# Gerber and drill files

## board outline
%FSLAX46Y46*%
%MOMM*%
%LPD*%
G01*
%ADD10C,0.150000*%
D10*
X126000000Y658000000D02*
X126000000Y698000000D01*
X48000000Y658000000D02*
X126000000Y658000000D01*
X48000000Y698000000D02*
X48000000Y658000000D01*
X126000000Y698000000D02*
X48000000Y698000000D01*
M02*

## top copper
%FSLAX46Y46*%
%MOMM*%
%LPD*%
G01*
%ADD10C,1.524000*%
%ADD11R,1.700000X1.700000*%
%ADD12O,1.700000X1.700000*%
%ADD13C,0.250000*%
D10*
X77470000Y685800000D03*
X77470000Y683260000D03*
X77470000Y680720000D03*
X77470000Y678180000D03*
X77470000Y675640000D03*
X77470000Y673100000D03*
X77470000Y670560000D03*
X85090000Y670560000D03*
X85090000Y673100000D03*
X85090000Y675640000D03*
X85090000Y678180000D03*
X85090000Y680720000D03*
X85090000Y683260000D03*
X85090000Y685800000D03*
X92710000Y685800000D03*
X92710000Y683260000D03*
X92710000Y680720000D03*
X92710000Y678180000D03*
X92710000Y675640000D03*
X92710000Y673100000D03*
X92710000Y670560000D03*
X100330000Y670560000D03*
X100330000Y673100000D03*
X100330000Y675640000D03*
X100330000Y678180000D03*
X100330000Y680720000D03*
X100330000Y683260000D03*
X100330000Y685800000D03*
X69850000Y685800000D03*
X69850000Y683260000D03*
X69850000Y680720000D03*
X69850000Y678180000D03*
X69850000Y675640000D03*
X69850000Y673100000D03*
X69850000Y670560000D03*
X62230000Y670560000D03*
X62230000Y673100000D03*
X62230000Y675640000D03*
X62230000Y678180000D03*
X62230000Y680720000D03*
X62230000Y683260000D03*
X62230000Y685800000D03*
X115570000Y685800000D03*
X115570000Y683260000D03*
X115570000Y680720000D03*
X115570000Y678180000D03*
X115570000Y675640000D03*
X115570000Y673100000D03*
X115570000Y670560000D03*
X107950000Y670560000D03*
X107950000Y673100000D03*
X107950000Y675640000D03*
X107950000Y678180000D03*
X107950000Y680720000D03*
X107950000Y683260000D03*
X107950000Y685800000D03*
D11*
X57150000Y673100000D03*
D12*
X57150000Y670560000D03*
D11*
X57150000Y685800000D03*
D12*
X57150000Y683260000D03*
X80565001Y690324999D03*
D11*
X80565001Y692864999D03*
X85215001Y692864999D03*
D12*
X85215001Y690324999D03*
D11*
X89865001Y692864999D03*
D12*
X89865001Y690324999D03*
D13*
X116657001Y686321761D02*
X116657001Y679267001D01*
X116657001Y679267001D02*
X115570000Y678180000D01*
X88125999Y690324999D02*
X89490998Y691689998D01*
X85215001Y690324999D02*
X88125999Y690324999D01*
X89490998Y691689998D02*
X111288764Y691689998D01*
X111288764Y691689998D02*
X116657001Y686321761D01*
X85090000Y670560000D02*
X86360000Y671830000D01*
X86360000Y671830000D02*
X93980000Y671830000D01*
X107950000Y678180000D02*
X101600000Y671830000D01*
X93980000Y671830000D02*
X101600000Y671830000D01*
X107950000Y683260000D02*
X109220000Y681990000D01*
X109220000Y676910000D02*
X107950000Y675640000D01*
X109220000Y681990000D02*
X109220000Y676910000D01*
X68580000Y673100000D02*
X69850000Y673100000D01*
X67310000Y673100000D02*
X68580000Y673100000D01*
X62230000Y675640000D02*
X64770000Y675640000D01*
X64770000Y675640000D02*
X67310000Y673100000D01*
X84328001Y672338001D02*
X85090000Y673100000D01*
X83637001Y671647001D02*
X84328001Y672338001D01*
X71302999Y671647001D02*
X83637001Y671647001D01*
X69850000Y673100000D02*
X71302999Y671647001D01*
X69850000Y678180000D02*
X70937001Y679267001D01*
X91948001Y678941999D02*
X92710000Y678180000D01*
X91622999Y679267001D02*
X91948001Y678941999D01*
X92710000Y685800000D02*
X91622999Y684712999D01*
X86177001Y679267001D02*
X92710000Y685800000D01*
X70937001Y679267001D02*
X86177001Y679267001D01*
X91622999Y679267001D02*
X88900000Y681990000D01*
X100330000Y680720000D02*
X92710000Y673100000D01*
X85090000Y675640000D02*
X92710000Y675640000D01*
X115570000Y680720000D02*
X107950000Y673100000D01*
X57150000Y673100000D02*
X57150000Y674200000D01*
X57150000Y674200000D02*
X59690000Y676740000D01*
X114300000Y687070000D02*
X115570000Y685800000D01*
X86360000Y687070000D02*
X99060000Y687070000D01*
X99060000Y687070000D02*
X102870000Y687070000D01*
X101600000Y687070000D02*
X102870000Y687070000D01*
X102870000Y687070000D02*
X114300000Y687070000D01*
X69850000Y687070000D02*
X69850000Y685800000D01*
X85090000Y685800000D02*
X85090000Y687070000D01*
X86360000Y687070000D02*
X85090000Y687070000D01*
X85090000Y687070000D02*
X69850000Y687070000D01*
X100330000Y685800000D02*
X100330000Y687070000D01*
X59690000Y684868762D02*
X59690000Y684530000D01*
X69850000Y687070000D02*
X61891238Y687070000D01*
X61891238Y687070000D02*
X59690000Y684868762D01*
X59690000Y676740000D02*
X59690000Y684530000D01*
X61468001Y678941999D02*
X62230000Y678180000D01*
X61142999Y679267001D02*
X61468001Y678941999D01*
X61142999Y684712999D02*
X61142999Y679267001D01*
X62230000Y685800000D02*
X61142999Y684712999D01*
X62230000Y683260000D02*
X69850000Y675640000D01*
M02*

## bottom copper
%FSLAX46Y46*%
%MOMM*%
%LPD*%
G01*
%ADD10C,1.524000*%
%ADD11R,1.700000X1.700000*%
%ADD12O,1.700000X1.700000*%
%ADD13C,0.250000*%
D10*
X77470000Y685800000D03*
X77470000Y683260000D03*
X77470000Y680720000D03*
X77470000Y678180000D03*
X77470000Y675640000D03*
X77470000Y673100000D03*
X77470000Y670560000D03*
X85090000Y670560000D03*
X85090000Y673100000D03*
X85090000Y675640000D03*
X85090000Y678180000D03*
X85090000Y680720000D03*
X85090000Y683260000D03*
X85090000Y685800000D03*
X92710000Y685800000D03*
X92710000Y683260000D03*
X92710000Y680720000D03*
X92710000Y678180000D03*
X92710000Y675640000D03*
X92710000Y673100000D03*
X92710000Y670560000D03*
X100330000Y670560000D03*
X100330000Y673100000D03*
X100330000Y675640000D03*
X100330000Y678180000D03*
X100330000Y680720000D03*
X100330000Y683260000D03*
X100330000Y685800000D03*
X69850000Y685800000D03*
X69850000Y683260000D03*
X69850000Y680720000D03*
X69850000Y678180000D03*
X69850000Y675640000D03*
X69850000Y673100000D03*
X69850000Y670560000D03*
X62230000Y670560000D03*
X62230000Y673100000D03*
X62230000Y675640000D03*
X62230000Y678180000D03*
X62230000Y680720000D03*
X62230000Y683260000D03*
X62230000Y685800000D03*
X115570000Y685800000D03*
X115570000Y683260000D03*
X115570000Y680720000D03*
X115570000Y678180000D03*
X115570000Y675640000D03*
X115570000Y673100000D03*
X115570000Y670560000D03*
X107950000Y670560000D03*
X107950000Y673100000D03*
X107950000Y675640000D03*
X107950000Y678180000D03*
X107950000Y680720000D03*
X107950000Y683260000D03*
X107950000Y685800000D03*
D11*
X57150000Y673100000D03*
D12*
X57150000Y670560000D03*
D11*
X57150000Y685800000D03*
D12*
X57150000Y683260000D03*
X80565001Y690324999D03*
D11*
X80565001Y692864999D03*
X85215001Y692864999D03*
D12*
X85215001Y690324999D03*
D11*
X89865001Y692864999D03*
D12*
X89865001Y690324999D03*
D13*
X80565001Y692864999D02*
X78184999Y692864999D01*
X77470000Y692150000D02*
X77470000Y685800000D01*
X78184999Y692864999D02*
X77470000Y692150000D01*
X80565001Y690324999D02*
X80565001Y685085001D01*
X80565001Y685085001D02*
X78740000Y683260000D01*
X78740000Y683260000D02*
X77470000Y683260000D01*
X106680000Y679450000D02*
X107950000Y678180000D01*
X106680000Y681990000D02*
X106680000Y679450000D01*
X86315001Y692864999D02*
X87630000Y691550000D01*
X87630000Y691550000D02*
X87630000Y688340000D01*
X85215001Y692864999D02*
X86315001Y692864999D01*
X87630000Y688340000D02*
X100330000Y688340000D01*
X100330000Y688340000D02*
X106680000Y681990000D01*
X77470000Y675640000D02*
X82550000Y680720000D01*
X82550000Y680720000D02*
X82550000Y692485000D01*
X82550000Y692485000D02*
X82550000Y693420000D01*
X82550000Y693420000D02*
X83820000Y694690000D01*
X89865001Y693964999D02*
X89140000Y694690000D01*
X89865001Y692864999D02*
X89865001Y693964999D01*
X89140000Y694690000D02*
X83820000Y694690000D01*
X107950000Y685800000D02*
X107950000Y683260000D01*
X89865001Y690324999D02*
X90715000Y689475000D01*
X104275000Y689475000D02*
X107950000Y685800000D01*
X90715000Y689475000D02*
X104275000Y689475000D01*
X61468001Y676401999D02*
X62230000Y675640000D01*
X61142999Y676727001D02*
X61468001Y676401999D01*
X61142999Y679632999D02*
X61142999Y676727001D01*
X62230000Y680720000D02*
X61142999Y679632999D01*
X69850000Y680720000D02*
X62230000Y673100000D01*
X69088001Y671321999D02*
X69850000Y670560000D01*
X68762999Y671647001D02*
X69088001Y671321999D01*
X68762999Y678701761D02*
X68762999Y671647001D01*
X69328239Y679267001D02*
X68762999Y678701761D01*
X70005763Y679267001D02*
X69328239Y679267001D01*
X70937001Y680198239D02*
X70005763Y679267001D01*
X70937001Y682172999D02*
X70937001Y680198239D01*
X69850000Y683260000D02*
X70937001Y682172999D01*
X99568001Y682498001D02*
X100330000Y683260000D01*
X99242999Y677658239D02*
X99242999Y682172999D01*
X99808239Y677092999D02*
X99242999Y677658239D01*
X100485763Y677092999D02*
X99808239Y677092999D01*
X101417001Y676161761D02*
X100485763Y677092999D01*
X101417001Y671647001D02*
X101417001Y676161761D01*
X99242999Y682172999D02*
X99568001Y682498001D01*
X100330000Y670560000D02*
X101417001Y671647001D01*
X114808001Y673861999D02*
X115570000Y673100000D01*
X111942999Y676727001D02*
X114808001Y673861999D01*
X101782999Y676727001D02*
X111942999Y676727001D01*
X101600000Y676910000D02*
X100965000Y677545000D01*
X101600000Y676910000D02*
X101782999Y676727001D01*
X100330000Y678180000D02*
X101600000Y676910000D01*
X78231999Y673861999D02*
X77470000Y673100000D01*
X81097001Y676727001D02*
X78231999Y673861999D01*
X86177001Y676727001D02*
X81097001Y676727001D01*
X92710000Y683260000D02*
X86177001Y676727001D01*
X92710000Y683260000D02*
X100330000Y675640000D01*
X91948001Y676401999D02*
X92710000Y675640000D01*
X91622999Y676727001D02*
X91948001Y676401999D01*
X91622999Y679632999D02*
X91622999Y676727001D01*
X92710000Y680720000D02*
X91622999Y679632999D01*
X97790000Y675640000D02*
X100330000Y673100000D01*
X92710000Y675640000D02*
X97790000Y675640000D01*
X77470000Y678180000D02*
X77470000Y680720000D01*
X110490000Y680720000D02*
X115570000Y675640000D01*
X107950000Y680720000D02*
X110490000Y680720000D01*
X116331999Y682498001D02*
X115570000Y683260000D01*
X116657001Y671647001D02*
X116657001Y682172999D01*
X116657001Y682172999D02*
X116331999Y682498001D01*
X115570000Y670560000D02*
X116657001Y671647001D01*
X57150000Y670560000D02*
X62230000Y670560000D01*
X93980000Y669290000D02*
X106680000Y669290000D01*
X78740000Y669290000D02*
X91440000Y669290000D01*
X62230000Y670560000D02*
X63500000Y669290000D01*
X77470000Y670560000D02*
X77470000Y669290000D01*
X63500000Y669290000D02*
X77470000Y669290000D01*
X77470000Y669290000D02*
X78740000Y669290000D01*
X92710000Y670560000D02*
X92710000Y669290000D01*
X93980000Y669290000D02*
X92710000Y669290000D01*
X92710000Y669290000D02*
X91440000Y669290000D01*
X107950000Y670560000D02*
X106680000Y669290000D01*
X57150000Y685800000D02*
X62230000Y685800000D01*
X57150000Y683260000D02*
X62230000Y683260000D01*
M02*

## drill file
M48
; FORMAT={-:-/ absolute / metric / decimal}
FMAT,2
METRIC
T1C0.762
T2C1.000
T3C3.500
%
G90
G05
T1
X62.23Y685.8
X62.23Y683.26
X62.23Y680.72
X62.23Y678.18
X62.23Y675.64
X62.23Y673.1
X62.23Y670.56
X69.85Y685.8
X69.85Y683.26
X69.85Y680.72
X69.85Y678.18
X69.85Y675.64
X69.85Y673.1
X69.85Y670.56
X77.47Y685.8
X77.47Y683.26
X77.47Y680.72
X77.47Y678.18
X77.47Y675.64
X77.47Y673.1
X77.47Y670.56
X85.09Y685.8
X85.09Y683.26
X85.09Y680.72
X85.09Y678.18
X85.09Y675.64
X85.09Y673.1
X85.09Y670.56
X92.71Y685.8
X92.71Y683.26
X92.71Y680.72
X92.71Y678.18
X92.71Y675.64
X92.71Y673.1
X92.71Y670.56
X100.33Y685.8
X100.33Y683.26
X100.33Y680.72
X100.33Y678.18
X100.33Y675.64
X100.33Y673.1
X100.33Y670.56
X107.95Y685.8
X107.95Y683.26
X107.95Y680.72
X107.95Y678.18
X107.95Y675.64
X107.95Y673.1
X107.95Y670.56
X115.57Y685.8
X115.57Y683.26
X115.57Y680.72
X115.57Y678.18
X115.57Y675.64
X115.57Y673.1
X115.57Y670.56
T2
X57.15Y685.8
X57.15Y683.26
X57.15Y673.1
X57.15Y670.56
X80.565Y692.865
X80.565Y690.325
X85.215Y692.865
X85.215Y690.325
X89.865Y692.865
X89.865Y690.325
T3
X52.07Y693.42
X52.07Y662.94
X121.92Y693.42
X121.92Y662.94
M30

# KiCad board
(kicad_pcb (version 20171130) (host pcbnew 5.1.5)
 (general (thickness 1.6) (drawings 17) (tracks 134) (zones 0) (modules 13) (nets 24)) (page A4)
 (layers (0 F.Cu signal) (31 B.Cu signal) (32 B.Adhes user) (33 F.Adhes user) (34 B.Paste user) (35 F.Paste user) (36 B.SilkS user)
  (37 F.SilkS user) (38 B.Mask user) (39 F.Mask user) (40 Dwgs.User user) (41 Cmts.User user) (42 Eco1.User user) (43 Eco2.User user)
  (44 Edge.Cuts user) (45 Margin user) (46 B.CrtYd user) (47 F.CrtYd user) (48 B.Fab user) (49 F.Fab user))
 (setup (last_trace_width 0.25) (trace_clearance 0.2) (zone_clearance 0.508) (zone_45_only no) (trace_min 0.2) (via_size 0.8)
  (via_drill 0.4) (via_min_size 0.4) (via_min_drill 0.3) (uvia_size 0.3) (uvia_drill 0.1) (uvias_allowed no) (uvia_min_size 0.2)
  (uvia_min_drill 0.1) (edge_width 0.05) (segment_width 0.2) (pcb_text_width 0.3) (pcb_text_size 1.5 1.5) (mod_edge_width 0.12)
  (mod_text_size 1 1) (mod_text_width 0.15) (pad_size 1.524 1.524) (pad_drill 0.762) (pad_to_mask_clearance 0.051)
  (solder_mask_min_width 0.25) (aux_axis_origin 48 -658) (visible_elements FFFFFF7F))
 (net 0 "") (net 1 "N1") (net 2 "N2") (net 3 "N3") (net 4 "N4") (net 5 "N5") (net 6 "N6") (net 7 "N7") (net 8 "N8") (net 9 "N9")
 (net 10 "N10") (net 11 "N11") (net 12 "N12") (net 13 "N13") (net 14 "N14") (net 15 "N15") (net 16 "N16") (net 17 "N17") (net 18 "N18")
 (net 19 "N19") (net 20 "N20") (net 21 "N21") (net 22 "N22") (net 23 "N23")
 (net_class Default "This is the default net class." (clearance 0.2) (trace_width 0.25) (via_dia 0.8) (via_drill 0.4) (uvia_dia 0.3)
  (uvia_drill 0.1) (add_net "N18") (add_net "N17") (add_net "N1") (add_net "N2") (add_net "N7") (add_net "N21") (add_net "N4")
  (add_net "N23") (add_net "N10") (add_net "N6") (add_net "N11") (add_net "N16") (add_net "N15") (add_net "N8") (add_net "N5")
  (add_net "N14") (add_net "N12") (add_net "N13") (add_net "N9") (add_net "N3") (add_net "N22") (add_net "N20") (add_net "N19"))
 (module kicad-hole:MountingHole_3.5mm (layer F.Cu) (at 121.92 -662.94)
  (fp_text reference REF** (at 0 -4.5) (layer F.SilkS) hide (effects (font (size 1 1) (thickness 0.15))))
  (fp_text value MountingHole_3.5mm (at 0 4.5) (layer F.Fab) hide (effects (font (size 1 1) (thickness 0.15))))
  (pad 1 np_thru_hole circle (at 0 0) (size 3.5 3.5) (drill 3.5) (layers *.Cu *.Mask)))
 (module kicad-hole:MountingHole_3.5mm (layer F.Cu) (at 52.07 -693.42)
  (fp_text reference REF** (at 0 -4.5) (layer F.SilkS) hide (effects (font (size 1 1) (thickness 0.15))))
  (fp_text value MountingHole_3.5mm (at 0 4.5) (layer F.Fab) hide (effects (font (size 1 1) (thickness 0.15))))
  (pad 1 np_thru_hole circle (at 0 0) (size 3.5 3.5) (drill 3.5) (layers *.Cu *.Mask)))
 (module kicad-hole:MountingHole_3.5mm (layer F.Cu) (at 52.07 -662.94)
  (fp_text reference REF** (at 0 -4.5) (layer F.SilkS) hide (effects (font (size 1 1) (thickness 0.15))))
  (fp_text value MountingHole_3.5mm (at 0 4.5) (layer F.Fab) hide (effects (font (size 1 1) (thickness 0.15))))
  (pad 1 np_thru_hole circle (at 0 0) (size 3.5 3.5) (drill 3.5) (layers *.Cu *.Mask)))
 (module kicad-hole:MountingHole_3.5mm (layer F.Cu) (at 121.92 -693.42)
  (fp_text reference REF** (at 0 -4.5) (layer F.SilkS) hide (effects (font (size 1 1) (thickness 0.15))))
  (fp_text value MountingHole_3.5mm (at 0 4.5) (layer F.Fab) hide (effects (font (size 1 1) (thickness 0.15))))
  (pad 1 np_thru_hole circle (at 0 0) (size 3.5 3.5) (drill 3.5) (layers *.Cu *.Mask)))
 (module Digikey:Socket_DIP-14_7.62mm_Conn (layer F.Cu) (at 77.47 -685.8)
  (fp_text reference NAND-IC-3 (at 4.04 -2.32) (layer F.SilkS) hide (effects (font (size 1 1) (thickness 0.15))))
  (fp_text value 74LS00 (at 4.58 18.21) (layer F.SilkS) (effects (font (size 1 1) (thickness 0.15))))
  (pad 1 thru_hole circle (at 0 0) (size 1.524 1.524) (drill 0.762) (layers *.Cu *.Mask) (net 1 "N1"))
  (pad 2 thru_hole circle (at 0 2.54) (size 1.524 1.524) (drill 0.762) (layers *.Cu *.Mask) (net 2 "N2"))
  (pad 3 thru_hole circle (at 0 5.08) (size 1.524 1.524) (drill 0.762) (layers *.Cu *.Mask) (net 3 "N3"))
  (pad 4 thru_hole circle (at 0 7.62) (size 1.524 1.524) (drill 0.762) (layers *.Cu *.Mask) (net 3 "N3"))
  (pad 5 thru_hole circle (at 0 10.16) (size 1.524 1.524) (drill 0.762) (layers *.Cu *.Mask) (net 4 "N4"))
  (pad 6 thru_hole circle (at 0 12.7) (size 1.524 1.524) (drill 0.762) (layers *.Cu *.Mask) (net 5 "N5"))
  (pad 7 thru_hole circle (at 0 15.24) (size 1.524 1.524) (drill 0.762) (layers *.Cu *.Mask) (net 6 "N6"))
  (pad 8 thru_hole circle (at 7.62 15.24) (size 1.524 1.524) (drill 0.762) (layers *.Cu *.Mask) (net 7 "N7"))
  (pad 9 thru_hole circle (at 7.62 12.7) (size 1.524 1.524) (drill 0.762) (layers *.Cu *.Mask) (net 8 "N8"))
  (pad 10 thru_hole circle (at 7.62 10.16) (size 1.524 1.524) (drill 0.762) (layers *.Cu *.Mask) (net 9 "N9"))
  (pad 11 thru_hole circle (at 7.62 7.62) (size 1.524 1.524) (drill 0.762) (layers *.Cu *.Mask))
  (pad 12 thru_hole circle (at 7.62 5.08) (size 1.524 1.524) (drill 0.762) (layers *.Cu *.Mask))
  (pad 13 thru_hole circle (at 7.62 2.54) (size 1.524 1.524) (drill 0.762) (layers *.Cu *.Mask))
  (pad 14 thru_hole circle (at 7.62 0) (size 1.524 1.524) (drill 0.762) (layers *.Cu *.Mask) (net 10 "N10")))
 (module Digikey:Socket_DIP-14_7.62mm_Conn (layer F.Cu) (at 92.71 -685.8)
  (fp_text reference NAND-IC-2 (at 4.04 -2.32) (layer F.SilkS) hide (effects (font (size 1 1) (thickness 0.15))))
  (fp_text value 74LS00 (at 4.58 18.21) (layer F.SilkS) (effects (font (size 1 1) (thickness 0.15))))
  (pad 1 thru_hole circle (at 0 0) (size 1.524 1.524) (drill 0.762) (layers *.Cu *.Mask) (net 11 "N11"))
  (pad 2 thru_hole circle (at 0 2.54) (size 1.524 1.524) (drill 0.762) (layers *.Cu *.Mask) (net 5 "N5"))
  (pad 3 thru_hole circle (at 0 5.08) (size 1.524 1.524) (drill 0.762) (layers *.Cu *.Mask) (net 9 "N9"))
  (pad 4 thru_hole circle (at 0 7.62) (size 1.524 1.524) (drill 0.762) (layers *.Cu *.Mask) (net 11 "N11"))
  (pad 5 thru_hole circle (at 0 10.16) (size 1.524 1.524) (drill 0.762) (layers *.Cu *.Mask) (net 9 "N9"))
  (pad 6 thru_hole circle (at 0 12.7) (size 1.524 1.524) (drill 0.762) (layers *.Cu *.Mask) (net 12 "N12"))
  (pad 7 thru_hole circle (at 0 15.24) (size 1.524 1.524) (drill 0.762) (layers *.Cu *.Mask) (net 6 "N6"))
  (pad 8 thru_hole circle (at 7.62 15.24) (size 1.524 1.524) (drill 0.762) (layers *.Cu *.Mask) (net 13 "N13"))
  (pad 9 thru_hole circle (at 7.62 12.7) (size 1.524 1.524) (drill 0.762) (layers *.Cu *.Mask) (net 9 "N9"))
  (pad 10 thru_hole circle (at 7.62 10.16) (size 1.524 1.524) (drill 0.762) (layers *.Cu *.Mask) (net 5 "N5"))
  (pad 11 thru_hole circle (at 7.62 7.62) (size 1.524 1.524) (drill 0.762) (layers *.Cu *.Mask) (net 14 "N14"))
  (pad 12 thru_hole circle (at 7.62 5.08) (size 1.524 1.524) (drill 0.762) (layers *.Cu *.Mask) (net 12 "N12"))
  (pad 13 thru_hole circle (at 7.62 2.54) (size 1.524 1.524) (drill 0.762) (layers *.Cu *.Mask) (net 13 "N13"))
  (pad 14 thru_hole circle (at 7.62 0) (size 1.524 1.524) (drill 0.762) (layers *.Cu *.Mask) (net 10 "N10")))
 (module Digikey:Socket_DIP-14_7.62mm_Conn (layer F.Cu) (at 62.23 -685.8)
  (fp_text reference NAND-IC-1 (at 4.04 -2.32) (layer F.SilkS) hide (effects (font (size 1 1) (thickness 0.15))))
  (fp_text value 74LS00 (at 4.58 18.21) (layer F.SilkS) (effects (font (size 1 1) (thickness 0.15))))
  (pad 14 thru_hole circle (at 7.62 0) (size 1.524 1.524) (drill 0.762) (layers *.Cu *.Mask) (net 10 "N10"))
  (pad 13 thru_hole circle (at 7.62 2.54) (size 1.524 1.524) (drill 0.762) (layers *.Cu *.Mask) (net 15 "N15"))
  (pad 12 thru_hole circle (at 7.62 5.08) (size 1.524 1.524) (drill 0.762) (layers *.Cu *.Mask) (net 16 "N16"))
  (pad 11 thru_hole circle (at 7.62 7.62) (size 1.524 1.524) (drill 0.762) (layers *.Cu *.Mask) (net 11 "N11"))
  (pad 10 thru_hole circle (at 7.62 10.16) (size 1.524 1.524) (drill 0.762) (layers *.Cu *.Mask) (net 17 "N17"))
  (pad 9 thru_hole circle (at 7.62 12.7) (size 1.524 1.524) (drill 0.762) (layers *.Cu *.Mask) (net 8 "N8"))
  (pad 8 thru_hole circle (at 7.62 15.24) (size 1.524 1.524) (drill 0.762) (layers *.Cu *.Mask) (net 15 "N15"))
  (pad 7 thru_hole circle (at 0 15.24) (size 1.524 1.524) (drill 0.762) (layers *.Cu *.Mask) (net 6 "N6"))
  (pad 6 thru_hole circle (at 0 12.7) (size 1.524 1.524) (drill 0.762) (layers *.Cu *.Mask) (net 16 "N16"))
  (pad 5 thru_hole circle (at 0 10.16) (size 1.524 1.524) (drill 0.762) (layers *.Cu *.Mask) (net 8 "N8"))
  (pad 4 thru_hole circle (at 0 7.62) (size 1.524 1.524) (drill 0.762) (layers *.Cu *.Mask) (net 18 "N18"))
  (pad 3 thru_hole circle (at 0 5.08) (size 1.524 1.524) (drill 0.762) (layers *.Cu *.Mask) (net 8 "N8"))
  (pad 2 thru_hole circle (at 0 2.54) (size 1.524 1.524) (drill 0.762) (layers *.Cu *.Mask) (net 17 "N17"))
  (pad 1 thru_hole circle (at 0 0) (size 1.524 1.524) (drill 0.762) (layers *.Cu *.Mask) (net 18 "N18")))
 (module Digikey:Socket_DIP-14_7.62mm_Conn (layer F.Cu) (at 107.95 -685.8)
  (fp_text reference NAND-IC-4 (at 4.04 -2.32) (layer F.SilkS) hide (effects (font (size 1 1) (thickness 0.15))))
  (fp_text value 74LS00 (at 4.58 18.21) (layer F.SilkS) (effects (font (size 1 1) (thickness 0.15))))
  (pad 14 thru_hole circle (at 7.62 0) (size 1.524 1.524) (drill 0.762) (layers *.Cu *.Mask) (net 10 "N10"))
  (pad 13 thru_hole circle (at 7.62 2.54) (size 1.524 1.524) (drill 0.762) (layers *.Cu *.Mask) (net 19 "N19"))
  (pad 12 thru_hole circle (at 7.62 5.08) (size 1.524 1.524) (drill 0.762) (layers *.Cu *.Mask) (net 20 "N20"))
  (pad 11 thru_hole circle (at 7.62 7.62) (size 1.524 1.524) (drill 0.762) (layers *.Cu *.Mask) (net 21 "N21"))
  (pad 10 thru_hole circle (at 7.62 10.16) (size 1.524 1.524) (drill 0.762) (layers *.Cu *.Mask) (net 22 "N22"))
  (pad 9 thru_hole circle (at 7.62 12.7) (size 1.524 1.524) (drill 0.762) (layers *.Cu *.Mask) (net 14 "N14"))
  (pad 8 thru_hole circle (at 7.62 15.24) (size 1.524 1.524) (drill 0.762) (layers *.Cu *.Mask) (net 19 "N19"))
  (pad 7 thru_hole circle (at 0 15.24) (size 1.524 1.524) (drill 0.762) (layers *.Cu *.Mask) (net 6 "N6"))
  (pad 6 thru_hole circle (at 0 12.7) (size 1.524 1.524) (drill 0.762) (layers *.Cu *.Mask) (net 20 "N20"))
  (pad 5 thru_hole circle (at 0 10.16) (size 1.524 1.524) (drill 0.762) (layers *.Cu *.Mask) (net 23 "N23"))
  (pad 4 thru_hole circle (at 0 7.62) (size 1.524 1.524) (drill 0.762) (layers *.Cu *.Mask) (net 7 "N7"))
  (pad 3 thru_hole circle (at 0 5.08) (size 1.524 1.524) (drill 0.762) (layers *.Cu *.Mask) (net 22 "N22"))
  (pad 2 thru_hole circle (at 0 2.54) (size 1.524 1.524) (drill 0.762) (layers *.Cu *.Mask) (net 23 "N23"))
  (pad 1 thru_hole circle (at 0 0) (size 1.524 1.524) (drill 0.762) (layers *.Cu *.Mask) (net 23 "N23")))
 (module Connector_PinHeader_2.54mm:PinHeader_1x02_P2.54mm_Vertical (layer F.Cu) (at 57.15 -673.1)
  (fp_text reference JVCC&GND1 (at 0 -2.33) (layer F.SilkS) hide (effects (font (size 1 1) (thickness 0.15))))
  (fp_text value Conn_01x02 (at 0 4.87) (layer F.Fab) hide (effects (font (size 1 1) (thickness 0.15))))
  (pad 1 thru_hole rect (at 0 0) (size 1.7 1.7) (drill 1) (layers *.Cu *.Mask) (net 10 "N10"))
  (pad 2 thru_hole oval (at 0 2.54) (size 1.7 1.7) (drill 1) (layers *.Cu *.Mask) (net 6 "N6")))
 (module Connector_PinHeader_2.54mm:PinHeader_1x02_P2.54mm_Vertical (layer F.Cu) (at 57.15 -685.8)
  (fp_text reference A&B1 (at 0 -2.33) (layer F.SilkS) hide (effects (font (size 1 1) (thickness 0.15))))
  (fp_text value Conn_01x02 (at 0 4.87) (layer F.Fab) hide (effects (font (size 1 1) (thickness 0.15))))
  (pad 1 thru_hole rect (at 0 0) (size 1.7 1.7) (drill 1) (layers *.Cu *.Mask) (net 18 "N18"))
  (pad 2 thru_hole oval (at 0 2.54) (size 1.7 1.7) (drill 1) (layers *.Cu *.Mask) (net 17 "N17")))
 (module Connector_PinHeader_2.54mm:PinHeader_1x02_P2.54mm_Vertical (layer F.Cu) (at 80.565001 -692.864999)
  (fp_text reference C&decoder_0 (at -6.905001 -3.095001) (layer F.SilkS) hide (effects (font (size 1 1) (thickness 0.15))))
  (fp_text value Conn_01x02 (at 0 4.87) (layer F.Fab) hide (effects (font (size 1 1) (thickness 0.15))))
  (pad 2 thru_hole oval (at 0 2.54) (size 1.7 1.7) (drill 1) (layers *.Cu *.Mask) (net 2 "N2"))
  (pad 1 thru_hole rect (at 0 0) (size 1.7 1.7) (drill 1) (layers *.Cu *.Mask) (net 1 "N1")))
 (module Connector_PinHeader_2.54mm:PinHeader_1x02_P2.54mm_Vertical (layer F.Cu) (at 85.215001 -692.864999)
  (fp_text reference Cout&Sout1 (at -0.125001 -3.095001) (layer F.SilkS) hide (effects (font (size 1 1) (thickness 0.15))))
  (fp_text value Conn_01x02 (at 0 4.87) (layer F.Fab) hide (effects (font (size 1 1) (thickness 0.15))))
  (pad 1 thru_hole rect (at 0 0) (size 1.7 1.7) (drill 1) (layers *.Cu *.Mask) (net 7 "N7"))
  (pad 2 thru_hole oval (at 0 2.54) (size 1.7 1.7) (drill 1) (layers *.Cu *.Mask) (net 21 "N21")))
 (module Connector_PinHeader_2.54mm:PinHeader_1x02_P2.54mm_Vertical (layer F.Cu) (at 89.865001 -692.864999)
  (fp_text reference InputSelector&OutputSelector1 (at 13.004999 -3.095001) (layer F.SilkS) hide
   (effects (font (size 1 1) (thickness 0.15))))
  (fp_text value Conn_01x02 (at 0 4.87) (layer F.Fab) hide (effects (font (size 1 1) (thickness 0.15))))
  (pad 1 thru_hole rect (at 0 0) (size 1.7 1.7) (drill 1) (layers *.Cu *.Mask) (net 4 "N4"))
  (pad 2 thru_hole oval (at 0 2.54) (size 1.7 1.7) (drill 1) (layers *.Cu *.Mask) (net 23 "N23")))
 (gr_line (start 126 -658) (end 126 -698) (layer Edge.Cuts) (width 0.15))
 (gr_line (start 48 -658) (end 126 -658) (layer Edge.Cuts) (width 0.15))
 (gr_line (start 48 -698) (end 48 -658) (layer Edge.Cuts) (width 0.15))
 (gr_line (start 126 -698) (end 48 -698) (layer Edge.Cuts) (width 0.15))
 (segment (start 80.565001 -692.864999) (end 78.184999 -692.864999) (width 0.25) (layer B.Cu) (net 1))
 (segment (start 77.47 -692.15) (end 77.47 -685.8) (width 0.25) (layer B.Cu) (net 1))
 (segment (start 78.184999 -692.864999) (end 77.47 -692.15) (width 0.25) (layer B.Cu) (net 1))
 (segment (start 80.565001 -690.324999) (end 80.565001 -685.085001) (width 0.25) (layer B.Cu) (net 2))
 (segment (start 80.565001 -685.085001) (end 78.74 -683.26) (width 0.25) (layer B.Cu) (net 2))
 (segment (start 78.74 -683.26) (end 77.47 -683.26) (width 0.25) (layer B.Cu) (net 2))
 (segment (start 116.657001 -686.321761) (end 116.657001 -679.267001) (width 0.25) (layer F.Cu) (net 21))
 (segment (start 116.657001 -679.267001) (end 115.57 -678.18) (width 0.25) (layer F.Cu) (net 21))
 (segment (start 88.125999 -690.324999) (end 89.490998 -691.689998) (width 0.25) (layer F.Cu) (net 21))
 (segment (start 85.215001 -690.324999) (end 88.125999 -690.324999) (width 0.25) (layer F.Cu) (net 21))
 (segment (start 89.490998 -691.689998) (end 111.288764 -691.689998) (width 0.25) (layer F.Cu) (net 21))
 (segment (start 111.288764 -691.689998) (end 116.657001 -686.321761) (width 0.25) (layer F.Cu) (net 21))
 (segment (start 85.09 -670.56) (end 86.36 -671.83) (width 0.25) (layer F.Cu) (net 7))
 (segment (start 86.36 -671.83) (end 93.98 -671.83) (width 0.25) (layer F.Cu) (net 7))
 (segment (start 107.95 -678.18) (end 101.6 -671.83) (width 0.25) (layer F.Cu) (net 7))
 (segment (start 93.98 -671.83) (end 101.6 -671.83) (width 0.25) (layer F.Cu) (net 7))
 (segment (start 106.68 -679.45) (end 107.95 -678.18) (width 0.25) (layer B.Cu) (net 7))
 (segment (start 106.68 -681.99) (end 106.68 -679.45) (width 0.25) (layer B.Cu) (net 7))
 (segment (start 86.315001 -692.864999) (end 87.63 -691.55) (width 0.25) (layer B.Cu) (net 7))
 (segment (start 87.63 -691.55) (end 87.63 -688.34) (width 0.25) (layer B.Cu) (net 7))
 (segment (start 85.215001 -692.864999) (end 86.315001 -692.864999) (width 0.25) (layer B.Cu) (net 7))
 (segment (start 87.63 -688.34) (end 100.33 -688.34) (width 0.25) (layer B.Cu) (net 7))
 (segment (start 100.33 -688.34) (end 106.68 -681.99) (width 0.25) (layer B.Cu) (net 7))
 (segment (start 77.47 -675.64) (end 82.55 -680.72) (width 0.25) (layer B.Cu) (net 4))
 (segment (start 82.55 -680.72) (end 82.55 -692.485) (width 0.25) (layer B.Cu) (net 4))
 (segment (start 82.55 -692.485) (end 82.55 -693.42) (width 0.25) (layer B.Cu) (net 4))
 (segment (start 82.55 -693.42) (end 83.82 -694.69) (width 0.25) (layer B.Cu) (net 4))
 (segment (start 89.865001 -693.964999) (end 89.14 -694.69) (width 0.25) (layer B.Cu) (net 4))
 (segment (start 89.865001 -692.864999) (end 89.865001 -693.964999) (width 0.25) (layer B.Cu) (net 4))
 (segment (start 89.14 -694.69) (end 83.82 -694.69) (width 0.25) (layer B.Cu) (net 4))
 (segment (start 107.95 -685.8) (end 107.95 -683.26) (width 0.25) (layer B.Cu) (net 23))
 (segment (start 89.865001 -690.324999) (end 90.715 -689.475) (width 0.25) (layer B.Cu) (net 23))
 (segment (start 104.275 -689.475) (end 107.95 -685.8) (width 0.25) (layer B.Cu) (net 23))
 (segment (start 90.715 -689.475) (end 104.275 -689.475) (width 0.25) (layer B.Cu) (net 23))
 (segment (start 107.95 -683.26) (end 109.22 -681.99) (width 0.25) (layer F.Cu) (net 23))
 (segment (start 109.22 -676.91) (end 107.95 -675.64) (width 0.25) (layer F.Cu) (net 23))
 (segment (start 109.22 -681.99) (end 109.22 -676.91) (width 0.25) (layer F.Cu) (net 23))
 (segment (start 61.468001 -676.401999) (end 62.23 -675.64) (width 0.25) (layer B.Cu) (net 8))
 (segment (start 61.142999 -676.727001) (end 61.468001 -676.401999) (width 0.25) (layer B.Cu) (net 8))
 (segment (start 61.142999 -679.632999) (end 61.142999 -676.727001) (width 0.25) (layer B.Cu) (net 8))
 (segment (start 62.23 -680.72) (end 61.142999 -679.632999) (width 0.25) (layer B.Cu) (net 8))
 (segment (start 68.58 -673.1) (end 69.85 -673.1) (width 0.25) (layer F.Cu) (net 8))
 (segment (start 67.31 -673.1) (end 68.58 -673.1) (width 0.25) (layer F.Cu) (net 8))
 (segment (start 62.23 -675.64) (end 64.77 -675.64) (width 0.25) (layer F.Cu) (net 8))
 (segment (start 64.77 -675.64) (end 67.31 -673.1) (width 0.25) (layer F.Cu) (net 8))
 (segment (start 84.328001 -672.338001) (end 85.09 -673.1) (width 0.25) (layer F.Cu) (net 8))
 (segment (start 83.637001 -671.647001) (end 84.328001 -672.338001) (width 0.25) (layer F.Cu) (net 8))
 (segment (start 71.302999 -671.647001) (end 83.637001 -671.647001) (width 0.25) (layer F.Cu) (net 8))
 (segment (start 69.85 -673.1) (end 71.302999 -671.647001) (width 0.25) (layer F.Cu) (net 8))
 (segment (start 69.85 -680.72) (end 62.23 -673.1) (width 0.25) (layer B.Cu) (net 16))
 (segment (start 69.088001 -671.321999) (end 69.85 -670.56) (width 0.25) (layer B.Cu) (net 15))
 (segment (start 68.762999 -671.647001) (end 69.088001 -671.321999) (width 0.25) (layer B.Cu) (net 15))
 (segment (start 68.762999 -678.701761) (end 68.762999 -671.647001) (width 0.25) (layer B.Cu) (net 15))
 (segment (start 69.328239 -679.267001) (end 68.762999 -678.701761) (width 0.25) (layer B.Cu) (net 15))
 (segment (start 70.005763 -679.267001) (end 69.328239 -679.267001) (width 0.25) (layer B.Cu) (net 15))
 (segment (start 70.937001 -680.198239) (end 70.005763 -679.267001) (width 0.25) (layer B.Cu) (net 15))
 (segment (start 70.937001 -682.172999) (end 70.937001 -680.198239) (width 0.25) (layer B.Cu) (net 15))
 (segment (start 69.85 -683.26) (end 70.937001 -682.172999) (width 0.25) (layer B.Cu) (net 15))
 (segment (start 69.85 -678.18) (end 70.937001 -679.267001) (width 0.25) (layer F.Cu) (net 11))
 (segment (start 91.948001 -678.941999) (end 92.71 -678.18) (width 0.25) (layer F.Cu) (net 11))
 (segment (start 91.622999 -679.267001) (end 91.948001 -678.941999) (width 0.25) (layer F.Cu) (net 11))
 (segment (start 92.71 -685.8) (end 91.622999 -684.712999) (width 0.25) (layer F.Cu) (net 11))
 (segment (start 86.177001 -679.267001) (end 92.71 -685.8) (width 0.25) (layer F.Cu) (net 11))
 (segment (start 70.937001 -679.267001) (end 86.177001 -679.267001) (width 0.25) (layer F.Cu) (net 11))
 (segment (start 91.622999 -679.267001) (end 88.9 -681.99) (width 0.25) (layer F.Cu) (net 11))
 (segment (start 99.568001 -682.498001) (end 100.33 -683.26) (width 0.25) (layer B.Cu) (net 13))
 (segment (start 99.242999 -677.658239) (end 99.242999 -682.172999) (width 0.25) (layer B.Cu) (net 13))
 (segment (start 99.808239 -677.092999) (end 99.242999 -677.658239) (width 0.25) (layer B.Cu) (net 13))
 (segment (start 100.485763 -677.092999) (end 99.808239 -677.092999) (width 0.25) (layer B.Cu) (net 13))
 (segment (start 101.417001 -676.161761) (end 100.485763 -677.092999) (width 0.25) (layer B.Cu) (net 13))
 (segment (start 101.417001 -671.647001) (end 101.417001 -676.161761) (width 0.25) (layer B.Cu) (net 13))
 (segment (start 99.242999 -682.172999) (end 99.568001 -682.498001) (width 0.25) (layer B.Cu) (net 13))
 (segment (start 100.33 -670.56) (end 101.417001 -671.647001) (width 0.25) (layer B.Cu) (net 13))
 (segment (start 100.33 -680.72) (end 92.71 -673.1) (width 0.25) (layer F.Cu) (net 12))
 (segment (start 114.808001 -673.861999) (end 115.57 -673.1) (width 0.25) (layer B.Cu) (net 14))
 (segment (start 111.942999 -676.727001) (end 114.808001 -673.861999) (width 0.25) (layer B.Cu) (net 14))
 (segment (start 101.782999 -676.727001) (end 111.942999 -676.727001) (width 0.25) (layer B.Cu) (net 14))
 (segment (start 101.6 -676.91) (end 100.965 -677.545) (width 0.25) (layer B.Cu) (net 14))
 (segment (start 101.6 -676.91) (end 101.782999 -676.727001) (width 0.25) (layer B.Cu) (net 14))
 (segment (start 100.33 -678.18) (end 101.6 -676.91) (width 0.25) (layer B.Cu) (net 14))
 (segment (start 78.231999 -673.861999) (end 77.47 -673.1) (width 0.25) (layer B.Cu) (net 5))
 (segment (start 81.097001 -676.727001) (end 78.231999 -673.861999) (width 0.25) (layer B.Cu) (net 5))
 (segment (start 86.177001 -676.727001) (end 81.097001 -676.727001) (width 0.25) (layer B.Cu) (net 5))
 (segment (start 92.71 -683.26) (end 86.177001 -676.727001) (width 0.25) (layer B.Cu) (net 5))
 (segment (start 92.71 -683.26) (end 100.33 -675.64) (width 0.25) (layer B.Cu) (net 5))
 (segment (start 85.09 -675.64) (end 92.71 -675.64) (width 0.25) (layer F.Cu) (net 9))
 (segment (start 91.948001 -676.401999) (end 92.71 -675.64) (width 0.25) (layer B.Cu) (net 9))
 (segment (start 91.622999 -676.727001) (end 91.948001 -676.401999) (width 0.25) (layer B.Cu) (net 9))
 (segment (start 91.622999 -679.632999) (end 91.622999 -676.727001) (width 0.25) (layer B.Cu) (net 9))
 (segment (start 92.71 -680.72) (end 91.622999 -679.632999) (width 0.25) (layer B.Cu) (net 9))
 (segment (start 97.79 -675.64) (end 100.33 -673.1) (width 0.25) (layer B.Cu) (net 9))
 (segment (start 92.71 -675.64) (end 97.79 -675.64) (width 0.25) (layer B.Cu) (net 9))
 (segment (start 77.47 -678.18) (end 77.47 -680.72) (width 0.25) (layer B.Cu) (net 3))
 (segment (start 110.49 -680.72) (end 115.57 -675.64) (width 0.25) (layer B.Cu) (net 22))
 (segment (start 107.95 -680.72) (end 110.49 -680.72) (width 0.25) (layer B.Cu) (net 22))
 (segment (start 115.57 -680.72) (end 107.95 -673.1) (width 0.25) (layer F.Cu) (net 20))
 (segment (start 116.331999 -682.498001) (end 115.57 -683.26) (width 0.25) (layer B.Cu) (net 19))
 (segment (start 116.657001 -671.647001) (end 116.657001 -682.172999) (width 0.25) (layer B.Cu) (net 19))
 (segment (start 116.657001 -682.172999) (end 116.331999 -682.498001) (width 0.25) (layer B.Cu) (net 19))
 (segment (start 115.57 -670.56) (end 116.657001 -671.647001) (width 0.25) (layer B.Cu) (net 19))
 (segment (start 57.15 -673.1) (end 57.15 -674.2) (width 0.25) (layer F.Cu) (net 10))
 (segment (start 57.15 -674.2) (end 59.69 -676.74) (width 0.25) (layer F.Cu) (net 10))
 (segment (start 114.3 -687.07) (end 115.57 -685.8) (width 0.25) (layer F.Cu) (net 10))
 (segment (start 86.36 -687.07) (end 99.06 -687.07) (width 0.25) (layer F.Cu) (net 10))
 (segment (start 99.06 -687.07) (end 102.87 -687.07) (width 0.25) (layer F.Cu) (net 10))
 (segment (start 101.6 -687.07) (end 102.87 -687.07) (width 0.25) (layer F.Cu) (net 10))
 (segment (start 102.87 -687.07) (end 114.3 -687.07) (width 0.25) (layer F.Cu) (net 10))
 (segment (start 69.85 -687.07) (end 69.85 -685.8) (width 0.25) (layer F.Cu) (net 10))
 (segment (start 85.09 -685.8) (end 85.09 -687.07) (width 0.25) (layer F.Cu) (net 10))
 (segment (start 86.36 -687.07) (end 85.09 -687.07) (width 0.25) (layer F.Cu) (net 10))
 (segment (start 85.09 -687.07) (end 69.85 -687.07) (width 0.25) (layer F.Cu) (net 10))
 (segment (start 100.33 -685.8) (end 100.33 -687.07) (width 0.25) (layer F.Cu) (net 10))
 (segment (start 59.69 -684.868762) (end 59.69 -684.53) (width 0.25) (layer F.Cu) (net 10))
 (segment (start 69.85 -687.07) (end 61.891238 -687.07) (width 0.25) (layer F.Cu) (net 10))
 (segment (start 61.891238 -687.07) (end 59.69 -684.868762) (width 0.25) (layer F.Cu) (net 10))
 (segment (start 59.69 -676.74) (end 59.69 -684.53) (width 0.25) (layer F.Cu) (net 10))
 (segment (start 57.15 -670.56) (end 62.23 -670.56) (width 0.25) (layer B.Cu) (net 6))
 (segment (start 93.98 -669.29) (end 106.68 -669.29) (width 0.25) (layer B.Cu) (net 6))
 (segment (start 78.74 -669.29) (end 91.44 -669.29) (width 0.25) (layer B.Cu) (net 6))
 (segment (start 62.23 -670.56) (end 63.5 -669.29) (width 0.25) (layer B.Cu) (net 6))
 (segment (start 77.47 -670.56) (end 77.47 -669.29) (width 0.25) (layer B.Cu) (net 6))
 (segment (start 63.5 -669.29) (end 77.47 -669.29) (width 0.25) (layer B.Cu) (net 6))
 (segment (start 77.47 -669.29) (end 78.74 -669.29) (width 0.25) (layer B.Cu) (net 6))
 (segment (start 92.71 -670.56) (end 92.71 -669.29) (width 0.25) (layer B.Cu) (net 6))
 (segment (start 93.98 -669.29) (end 92.71 -669.29) (width 0.25) (layer B.Cu) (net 6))
 (segment (start 92.71 -669.29) (end 91.44 -669.29) (width 0.25) (layer B.Cu) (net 6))
 (segment (start 107.95 -670.56) (end 106.68 -669.29) (width 0.25) (layer B.Cu) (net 6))
 (segment (start 57.15 -685.8) (end 62.23 -685.8) (width 0.25) (layer B.Cu) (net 18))
 (segment (start 61.468001 -678.941999) (end 62.23 -678.18) (width 0.25) (layer F.Cu) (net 18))
 (segment (start 61.142999 -679.267001) (end 61.468001 -678.941999) (width 0.25) (layer F.Cu) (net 18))
 (segment (start 61.142999 -684.712999) (end 61.142999 -679.267001) (width 0.25) (layer F.Cu) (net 18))
 (segment (start 62.23 -685.8) (end 61.142999 -684.712999) (width 0.25) (layer F.Cu) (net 18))
 (segment (start 57.15 -683.26) (end 62.23 -683.26) (width 0.25) (layer B.Cu) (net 17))
 (segment (start 62.23 -683.26) (end 69.85 -675.64) (width 0.25) (layer F.Cu) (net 17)))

